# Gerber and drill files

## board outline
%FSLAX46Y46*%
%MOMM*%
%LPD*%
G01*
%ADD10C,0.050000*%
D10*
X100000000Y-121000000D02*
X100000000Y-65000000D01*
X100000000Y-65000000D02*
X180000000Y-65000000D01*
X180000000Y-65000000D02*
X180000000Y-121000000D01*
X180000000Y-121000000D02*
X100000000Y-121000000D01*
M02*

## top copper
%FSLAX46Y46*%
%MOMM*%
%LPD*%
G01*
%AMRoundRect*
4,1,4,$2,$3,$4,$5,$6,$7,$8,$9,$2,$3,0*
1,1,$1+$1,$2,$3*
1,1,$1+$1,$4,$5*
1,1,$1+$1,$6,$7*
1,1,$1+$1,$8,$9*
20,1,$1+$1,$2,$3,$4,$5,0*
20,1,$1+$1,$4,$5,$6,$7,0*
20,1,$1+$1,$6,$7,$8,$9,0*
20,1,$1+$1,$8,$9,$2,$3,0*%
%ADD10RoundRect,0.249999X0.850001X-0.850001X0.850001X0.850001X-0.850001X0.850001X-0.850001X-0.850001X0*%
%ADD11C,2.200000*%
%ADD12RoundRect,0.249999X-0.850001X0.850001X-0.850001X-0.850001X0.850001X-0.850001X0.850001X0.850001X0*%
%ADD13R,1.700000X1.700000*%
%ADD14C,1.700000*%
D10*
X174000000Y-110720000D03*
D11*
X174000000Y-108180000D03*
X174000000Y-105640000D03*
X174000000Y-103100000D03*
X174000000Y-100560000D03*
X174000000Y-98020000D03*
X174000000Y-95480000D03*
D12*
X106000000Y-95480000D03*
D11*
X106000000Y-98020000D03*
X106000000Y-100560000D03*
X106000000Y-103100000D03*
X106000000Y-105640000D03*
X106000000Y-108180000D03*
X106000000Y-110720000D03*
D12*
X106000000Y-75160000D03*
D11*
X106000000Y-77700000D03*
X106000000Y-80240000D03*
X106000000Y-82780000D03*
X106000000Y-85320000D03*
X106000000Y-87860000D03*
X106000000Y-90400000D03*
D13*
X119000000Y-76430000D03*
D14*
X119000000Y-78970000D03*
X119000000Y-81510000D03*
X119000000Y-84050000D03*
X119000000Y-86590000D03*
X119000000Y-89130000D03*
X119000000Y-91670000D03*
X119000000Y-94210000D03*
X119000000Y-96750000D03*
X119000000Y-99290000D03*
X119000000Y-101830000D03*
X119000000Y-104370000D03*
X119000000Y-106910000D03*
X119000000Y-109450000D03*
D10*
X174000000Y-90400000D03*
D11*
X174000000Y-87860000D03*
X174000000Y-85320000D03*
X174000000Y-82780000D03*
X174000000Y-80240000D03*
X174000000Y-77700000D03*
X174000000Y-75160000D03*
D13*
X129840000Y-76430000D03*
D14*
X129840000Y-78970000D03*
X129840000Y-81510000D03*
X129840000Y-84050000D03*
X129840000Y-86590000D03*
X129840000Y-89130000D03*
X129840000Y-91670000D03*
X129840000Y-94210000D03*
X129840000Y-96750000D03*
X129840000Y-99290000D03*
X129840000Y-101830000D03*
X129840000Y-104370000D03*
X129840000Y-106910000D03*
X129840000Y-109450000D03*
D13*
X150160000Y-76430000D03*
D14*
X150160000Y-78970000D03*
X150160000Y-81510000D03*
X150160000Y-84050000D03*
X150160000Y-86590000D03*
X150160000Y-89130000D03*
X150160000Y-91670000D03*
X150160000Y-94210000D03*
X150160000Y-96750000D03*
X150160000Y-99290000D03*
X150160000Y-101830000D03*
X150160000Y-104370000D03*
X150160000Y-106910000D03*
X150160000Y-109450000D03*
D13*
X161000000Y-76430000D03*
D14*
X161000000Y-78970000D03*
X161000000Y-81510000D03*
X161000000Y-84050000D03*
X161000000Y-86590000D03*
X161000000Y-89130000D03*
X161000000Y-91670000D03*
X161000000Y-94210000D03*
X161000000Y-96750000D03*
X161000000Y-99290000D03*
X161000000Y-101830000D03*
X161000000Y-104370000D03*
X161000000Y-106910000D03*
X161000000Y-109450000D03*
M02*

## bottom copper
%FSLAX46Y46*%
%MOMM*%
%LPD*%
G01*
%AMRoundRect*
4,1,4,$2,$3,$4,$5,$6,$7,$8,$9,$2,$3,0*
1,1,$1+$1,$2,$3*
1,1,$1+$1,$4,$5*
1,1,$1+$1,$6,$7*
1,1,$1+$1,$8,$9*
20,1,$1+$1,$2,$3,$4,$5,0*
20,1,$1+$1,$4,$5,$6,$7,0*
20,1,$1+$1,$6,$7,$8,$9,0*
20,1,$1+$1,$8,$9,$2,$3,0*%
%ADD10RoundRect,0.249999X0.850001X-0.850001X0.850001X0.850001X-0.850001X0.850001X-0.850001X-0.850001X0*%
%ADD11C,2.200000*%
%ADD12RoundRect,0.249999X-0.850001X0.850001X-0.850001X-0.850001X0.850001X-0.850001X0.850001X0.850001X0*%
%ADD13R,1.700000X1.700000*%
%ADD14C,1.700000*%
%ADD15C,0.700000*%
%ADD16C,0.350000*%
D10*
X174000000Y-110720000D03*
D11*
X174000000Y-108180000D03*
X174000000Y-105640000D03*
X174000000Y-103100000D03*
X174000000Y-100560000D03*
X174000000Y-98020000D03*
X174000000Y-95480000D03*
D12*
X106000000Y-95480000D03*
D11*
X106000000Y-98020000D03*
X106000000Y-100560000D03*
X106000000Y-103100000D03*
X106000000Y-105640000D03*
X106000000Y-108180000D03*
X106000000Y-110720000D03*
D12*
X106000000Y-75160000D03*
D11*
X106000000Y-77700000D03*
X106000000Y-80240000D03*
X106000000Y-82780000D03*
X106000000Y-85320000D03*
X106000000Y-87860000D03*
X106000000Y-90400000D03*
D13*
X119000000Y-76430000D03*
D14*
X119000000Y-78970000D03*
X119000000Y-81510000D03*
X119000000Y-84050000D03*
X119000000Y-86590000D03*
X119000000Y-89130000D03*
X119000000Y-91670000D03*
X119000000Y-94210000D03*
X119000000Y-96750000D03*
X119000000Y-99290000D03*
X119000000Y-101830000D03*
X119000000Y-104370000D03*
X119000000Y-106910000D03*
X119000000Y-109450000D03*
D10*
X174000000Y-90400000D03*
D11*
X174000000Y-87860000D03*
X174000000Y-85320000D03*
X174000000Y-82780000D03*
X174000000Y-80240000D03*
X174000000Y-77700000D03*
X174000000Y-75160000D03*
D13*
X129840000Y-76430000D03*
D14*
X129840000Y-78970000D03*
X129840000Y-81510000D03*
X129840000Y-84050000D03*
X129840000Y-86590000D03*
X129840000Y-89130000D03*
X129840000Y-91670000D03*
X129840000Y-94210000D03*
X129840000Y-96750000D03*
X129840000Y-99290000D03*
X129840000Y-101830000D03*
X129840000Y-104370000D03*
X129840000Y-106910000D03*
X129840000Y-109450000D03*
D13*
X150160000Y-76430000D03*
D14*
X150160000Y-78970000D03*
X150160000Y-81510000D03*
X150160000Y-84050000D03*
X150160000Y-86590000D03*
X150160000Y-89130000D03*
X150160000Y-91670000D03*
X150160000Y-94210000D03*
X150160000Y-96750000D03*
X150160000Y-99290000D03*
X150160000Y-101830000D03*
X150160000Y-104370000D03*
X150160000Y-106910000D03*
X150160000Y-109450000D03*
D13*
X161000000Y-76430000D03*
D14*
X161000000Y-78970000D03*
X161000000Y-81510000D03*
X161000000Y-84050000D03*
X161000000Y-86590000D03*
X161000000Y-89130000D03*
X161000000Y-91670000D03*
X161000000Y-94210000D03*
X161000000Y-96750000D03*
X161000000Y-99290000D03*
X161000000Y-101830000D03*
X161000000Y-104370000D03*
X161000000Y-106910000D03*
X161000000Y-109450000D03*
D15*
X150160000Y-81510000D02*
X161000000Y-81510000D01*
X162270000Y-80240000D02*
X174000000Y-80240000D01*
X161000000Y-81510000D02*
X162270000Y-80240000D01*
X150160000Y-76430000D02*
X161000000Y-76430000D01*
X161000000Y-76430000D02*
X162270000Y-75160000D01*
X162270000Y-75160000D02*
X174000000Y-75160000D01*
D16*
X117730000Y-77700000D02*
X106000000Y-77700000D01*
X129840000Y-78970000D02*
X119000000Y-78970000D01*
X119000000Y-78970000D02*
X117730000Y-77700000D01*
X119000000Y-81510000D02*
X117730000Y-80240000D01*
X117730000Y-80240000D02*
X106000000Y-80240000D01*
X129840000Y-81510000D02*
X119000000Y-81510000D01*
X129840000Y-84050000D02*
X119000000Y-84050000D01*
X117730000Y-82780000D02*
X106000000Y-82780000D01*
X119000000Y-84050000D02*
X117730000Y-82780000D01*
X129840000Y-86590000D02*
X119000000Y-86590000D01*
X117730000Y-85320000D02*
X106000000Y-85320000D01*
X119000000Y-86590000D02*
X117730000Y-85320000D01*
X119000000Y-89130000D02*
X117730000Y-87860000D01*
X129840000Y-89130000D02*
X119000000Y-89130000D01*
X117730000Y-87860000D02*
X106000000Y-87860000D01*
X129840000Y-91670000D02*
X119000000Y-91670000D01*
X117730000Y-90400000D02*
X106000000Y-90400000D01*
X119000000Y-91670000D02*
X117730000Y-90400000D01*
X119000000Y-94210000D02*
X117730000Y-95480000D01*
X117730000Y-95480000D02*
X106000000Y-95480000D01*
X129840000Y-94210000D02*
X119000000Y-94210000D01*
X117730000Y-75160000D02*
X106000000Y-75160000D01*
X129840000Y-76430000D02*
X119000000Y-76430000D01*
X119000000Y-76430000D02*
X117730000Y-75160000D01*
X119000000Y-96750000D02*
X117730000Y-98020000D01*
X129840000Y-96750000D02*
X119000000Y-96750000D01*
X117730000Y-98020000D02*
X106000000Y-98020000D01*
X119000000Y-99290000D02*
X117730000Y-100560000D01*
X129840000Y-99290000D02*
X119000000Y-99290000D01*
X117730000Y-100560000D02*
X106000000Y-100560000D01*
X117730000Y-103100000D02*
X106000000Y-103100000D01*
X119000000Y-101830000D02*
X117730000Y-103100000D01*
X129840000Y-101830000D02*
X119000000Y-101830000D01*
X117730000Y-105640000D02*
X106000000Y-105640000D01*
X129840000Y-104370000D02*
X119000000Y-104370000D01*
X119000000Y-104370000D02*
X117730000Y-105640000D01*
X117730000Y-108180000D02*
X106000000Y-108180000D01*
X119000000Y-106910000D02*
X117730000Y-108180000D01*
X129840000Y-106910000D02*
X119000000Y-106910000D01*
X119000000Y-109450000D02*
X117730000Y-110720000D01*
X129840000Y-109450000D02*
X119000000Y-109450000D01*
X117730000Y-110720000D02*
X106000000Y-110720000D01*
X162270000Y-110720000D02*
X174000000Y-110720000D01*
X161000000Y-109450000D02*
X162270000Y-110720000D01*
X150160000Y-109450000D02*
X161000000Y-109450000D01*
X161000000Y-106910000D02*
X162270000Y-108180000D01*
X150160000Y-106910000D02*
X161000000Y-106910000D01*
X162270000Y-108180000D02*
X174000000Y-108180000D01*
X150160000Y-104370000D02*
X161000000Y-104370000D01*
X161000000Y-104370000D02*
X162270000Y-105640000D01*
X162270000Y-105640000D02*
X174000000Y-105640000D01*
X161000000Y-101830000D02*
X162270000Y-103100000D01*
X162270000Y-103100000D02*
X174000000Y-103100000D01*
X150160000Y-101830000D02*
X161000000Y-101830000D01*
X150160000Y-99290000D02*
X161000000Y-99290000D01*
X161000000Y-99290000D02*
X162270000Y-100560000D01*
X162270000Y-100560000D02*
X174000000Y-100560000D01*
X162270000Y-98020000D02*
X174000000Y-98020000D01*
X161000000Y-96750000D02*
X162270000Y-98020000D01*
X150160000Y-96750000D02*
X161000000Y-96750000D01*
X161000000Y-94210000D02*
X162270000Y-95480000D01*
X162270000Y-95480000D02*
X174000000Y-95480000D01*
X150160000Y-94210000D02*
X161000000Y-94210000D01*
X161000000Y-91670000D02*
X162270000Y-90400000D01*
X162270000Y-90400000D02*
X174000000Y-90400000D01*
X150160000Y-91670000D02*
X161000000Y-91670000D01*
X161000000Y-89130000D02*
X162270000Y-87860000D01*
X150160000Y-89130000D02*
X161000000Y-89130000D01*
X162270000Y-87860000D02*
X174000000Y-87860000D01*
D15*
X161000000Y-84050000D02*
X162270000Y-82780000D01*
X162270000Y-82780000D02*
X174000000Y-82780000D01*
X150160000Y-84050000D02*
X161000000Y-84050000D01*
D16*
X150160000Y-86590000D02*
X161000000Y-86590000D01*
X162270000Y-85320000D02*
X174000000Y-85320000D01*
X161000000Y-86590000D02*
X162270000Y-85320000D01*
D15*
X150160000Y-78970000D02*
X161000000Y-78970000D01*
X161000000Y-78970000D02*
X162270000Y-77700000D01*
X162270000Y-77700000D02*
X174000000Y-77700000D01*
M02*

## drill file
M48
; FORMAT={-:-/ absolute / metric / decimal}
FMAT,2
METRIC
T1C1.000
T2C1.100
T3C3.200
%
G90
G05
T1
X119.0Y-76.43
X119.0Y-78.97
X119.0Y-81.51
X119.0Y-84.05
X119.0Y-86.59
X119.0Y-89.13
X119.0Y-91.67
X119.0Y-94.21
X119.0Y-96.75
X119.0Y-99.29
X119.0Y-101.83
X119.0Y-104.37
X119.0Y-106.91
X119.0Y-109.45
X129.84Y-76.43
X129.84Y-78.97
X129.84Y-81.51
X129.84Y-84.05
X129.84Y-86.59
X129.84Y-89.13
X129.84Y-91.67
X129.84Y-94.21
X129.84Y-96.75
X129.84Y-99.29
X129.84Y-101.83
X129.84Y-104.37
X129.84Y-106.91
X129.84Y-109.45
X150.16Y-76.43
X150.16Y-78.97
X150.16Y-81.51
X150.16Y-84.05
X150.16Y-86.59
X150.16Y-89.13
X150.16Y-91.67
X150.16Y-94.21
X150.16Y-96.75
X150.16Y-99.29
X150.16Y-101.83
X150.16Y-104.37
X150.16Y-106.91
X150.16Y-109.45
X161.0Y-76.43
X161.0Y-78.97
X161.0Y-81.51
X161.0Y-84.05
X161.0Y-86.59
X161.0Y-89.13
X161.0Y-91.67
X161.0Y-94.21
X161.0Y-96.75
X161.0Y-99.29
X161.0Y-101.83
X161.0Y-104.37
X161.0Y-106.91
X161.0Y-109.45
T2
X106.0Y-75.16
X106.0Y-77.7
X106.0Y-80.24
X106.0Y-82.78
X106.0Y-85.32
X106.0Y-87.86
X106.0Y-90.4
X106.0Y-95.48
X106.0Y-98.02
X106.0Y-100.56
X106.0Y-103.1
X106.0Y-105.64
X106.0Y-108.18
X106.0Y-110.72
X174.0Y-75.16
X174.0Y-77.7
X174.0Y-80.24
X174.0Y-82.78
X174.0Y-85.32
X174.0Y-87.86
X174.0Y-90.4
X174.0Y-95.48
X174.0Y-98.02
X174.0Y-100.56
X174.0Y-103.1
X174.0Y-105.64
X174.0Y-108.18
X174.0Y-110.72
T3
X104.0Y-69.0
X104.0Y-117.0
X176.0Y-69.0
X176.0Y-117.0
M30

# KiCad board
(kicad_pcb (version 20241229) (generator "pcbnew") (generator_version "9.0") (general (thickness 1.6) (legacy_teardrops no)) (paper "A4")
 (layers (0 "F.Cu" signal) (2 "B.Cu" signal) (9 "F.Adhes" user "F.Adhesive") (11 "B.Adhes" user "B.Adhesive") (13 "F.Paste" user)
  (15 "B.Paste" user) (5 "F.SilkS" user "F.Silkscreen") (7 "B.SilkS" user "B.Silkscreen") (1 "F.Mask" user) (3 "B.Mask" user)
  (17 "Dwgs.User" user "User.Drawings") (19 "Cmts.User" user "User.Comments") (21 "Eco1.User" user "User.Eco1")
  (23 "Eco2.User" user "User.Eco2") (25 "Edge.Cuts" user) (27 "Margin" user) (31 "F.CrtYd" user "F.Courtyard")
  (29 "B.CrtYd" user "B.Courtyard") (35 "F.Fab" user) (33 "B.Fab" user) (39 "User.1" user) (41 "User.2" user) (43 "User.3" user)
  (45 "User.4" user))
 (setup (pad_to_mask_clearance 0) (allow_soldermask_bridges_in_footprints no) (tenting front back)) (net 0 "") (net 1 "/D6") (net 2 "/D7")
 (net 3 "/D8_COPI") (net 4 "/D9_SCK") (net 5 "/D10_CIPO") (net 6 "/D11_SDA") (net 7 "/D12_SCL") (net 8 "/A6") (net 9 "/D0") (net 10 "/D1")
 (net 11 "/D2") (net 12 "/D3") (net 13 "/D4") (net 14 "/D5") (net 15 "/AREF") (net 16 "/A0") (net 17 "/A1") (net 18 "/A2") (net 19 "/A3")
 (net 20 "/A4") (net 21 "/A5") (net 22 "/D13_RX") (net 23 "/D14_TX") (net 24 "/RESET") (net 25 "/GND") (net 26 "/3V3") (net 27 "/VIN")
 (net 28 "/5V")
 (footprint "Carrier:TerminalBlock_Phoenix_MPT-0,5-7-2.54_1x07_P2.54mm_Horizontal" (layer "F.Cu") (at 174 110.72 90)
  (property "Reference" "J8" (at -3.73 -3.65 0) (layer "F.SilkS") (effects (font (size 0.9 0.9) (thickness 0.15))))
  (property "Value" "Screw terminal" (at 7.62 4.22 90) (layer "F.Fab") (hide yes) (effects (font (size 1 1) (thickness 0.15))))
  (pad "1" thru_hole roundrect (at 0 0 90) (size 2.2 2.2) (drill 1.1) (layers "*.Cu" "*.Mask") (remove_unused_layers no)
   (roundrect_rratio 0.113636) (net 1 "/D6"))
  (pad "2" thru_hole circle (at 2.54 0 90) (size 2.2 2.2) (drill 1.1) (layers "*.Cu" "*.Mask") (remove_unused_layers no) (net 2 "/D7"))
  (pad "3" thru_hole circle (at 5.08 0 90) (size 2.2 2.2) (drill 1.1) (layers "*.Cu" "*.Mask") (remove_unused_layers no) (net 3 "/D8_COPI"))
  (pad "4" thru_hole circle (at 7.62 0 90) (size 2.2 2.2) (drill 1.1) (layers "*.Cu" "*.Mask") (remove_unused_layers no) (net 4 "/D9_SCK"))
  (pad "5" thru_hole circle (at 10.16 0 90) (size 2.2 2.2) (drill 1.1) (layers "*.Cu" "*.Mask") (remove_unused_layers no)
   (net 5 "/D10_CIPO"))
  (pad "6" thru_hole circle (at 12.7 0 90) (size 2.2 2.2) (drill 1.1) (layers "*.Cu" "*.Mask") (remove_unused_layers no) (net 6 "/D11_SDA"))
  (pad "7" thru_hole circle (at 15.24 0 90) (size 2.2 2.2) (drill 1.1) (layers "*.Cu" "*.Mask") (remove_unused_layers no) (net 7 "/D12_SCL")))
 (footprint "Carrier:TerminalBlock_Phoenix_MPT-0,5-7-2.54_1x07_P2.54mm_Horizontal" (layer "F.Cu") (at 106 95.48 -90)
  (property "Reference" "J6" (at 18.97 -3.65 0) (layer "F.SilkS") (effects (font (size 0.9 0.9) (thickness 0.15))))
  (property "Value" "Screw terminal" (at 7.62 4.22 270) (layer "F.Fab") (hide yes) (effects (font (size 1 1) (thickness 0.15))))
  (pad "1" thru_hole roundrect (at 0 0 270) (size 2.2 2.2) (drill 1.1) (layers "*.Cu" "*.Mask") (remove_unused_layers no)
   (roundrect_rratio 0.113636) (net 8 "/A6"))
  (pad "2" thru_hole circle (at 2.54 0 270) (size 2.2 2.2) (drill 1.1) (layers "*.Cu" "*.Mask") (remove_unused_layers no) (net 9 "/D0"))
  (pad "3" thru_hole circle (at 5.08 0 270) (size 2.2 2.2) (drill 1.1) (layers "*.Cu" "*.Mask") (remove_unused_layers no) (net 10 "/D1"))
  (pad "4" thru_hole circle (at 7.62 0 270) (size 2.2 2.2) (drill 1.1) (layers "*.Cu" "*.Mask") (remove_unused_layers no) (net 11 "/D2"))
  (pad "5" thru_hole circle (at 10.16 0 270) (size 2.2 2.2) (drill 1.1) (layers "*.Cu" "*.Mask") (remove_unused_layers no) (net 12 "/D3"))
  (pad "6" thru_hole circle (at 12.7 0 270) (size 2.2 2.2) (drill 1.1) (layers "*.Cu" "*.Mask") (remove_unused_layers no) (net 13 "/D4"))
  (pad "7" thru_hole circle (at 15.24 0 270) (size 2.2 2.2) (drill 1.1) (layers "*.Cu" "*.Mask") (remove_unused_layers no) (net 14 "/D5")))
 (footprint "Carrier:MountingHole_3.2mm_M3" (layer "F.Cu") (at 176 117)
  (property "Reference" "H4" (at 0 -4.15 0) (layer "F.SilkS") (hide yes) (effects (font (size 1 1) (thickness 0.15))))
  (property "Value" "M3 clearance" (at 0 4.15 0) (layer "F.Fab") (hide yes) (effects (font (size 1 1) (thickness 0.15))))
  (pad "" np_thru_hole circle (at 0 0) (size 3.2 3.2) (drill 3.2) (layers "*.Cu" "*.Mask")))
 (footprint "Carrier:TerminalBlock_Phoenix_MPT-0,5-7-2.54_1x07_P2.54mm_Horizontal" (layer "F.Cu") (at 106 75.16 -90)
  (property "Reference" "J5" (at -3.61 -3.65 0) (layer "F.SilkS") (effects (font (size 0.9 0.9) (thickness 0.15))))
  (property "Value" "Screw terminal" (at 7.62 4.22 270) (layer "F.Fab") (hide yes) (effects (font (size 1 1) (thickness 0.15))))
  (pad "1" thru_hole roundrect (at 0 0 270) (size 2.2 2.2) (drill 1.1) (layers "*.Cu" "*.Mask") (remove_unused_layers no)
   (roundrect_rratio 0.113636) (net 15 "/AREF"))
  (pad "2" thru_hole circle (at 2.54 0 270) (size 2.2 2.2) (drill 1.1) (layers "*.Cu" "*.Mask") (remove_unused_layers no) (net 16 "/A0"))
  (pad "3" thru_hole circle (at 5.08 0 270) (size 2.2 2.2) (drill 1.1) (layers "*.Cu" "*.Mask") (remove_unused_layers no) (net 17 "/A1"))
  (pad "4" thru_hole circle (at 7.62 0 270) (size 2.2 2.2) (drill 1.1) (layers "*.Cu" "*.Mask") (remove_unused_layers no) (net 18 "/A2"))
  (pad "5" thru_hole circle (at 10.16 0 270) (size 2.2 2.2) (drill 1.1) (layers "*.Cu" "*.Mask") (remove_unused_layers no) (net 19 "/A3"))
  (pad "6" thru_hole circle (at 12.7 0 270) (size 2.2 2.2) (drill 1.1) (layers "*.Cu" "*.Mask") (remove_unused_layers no) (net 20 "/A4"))
  (pad "7" thru_hole circle (at 15.24 0 270) (size 2.2 2.2) (drill 1.1) (layers "*.Cu" "*.Mask") (remove_unused_layers no) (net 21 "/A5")))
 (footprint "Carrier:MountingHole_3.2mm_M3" (layer "F.Cu") (at 176 69)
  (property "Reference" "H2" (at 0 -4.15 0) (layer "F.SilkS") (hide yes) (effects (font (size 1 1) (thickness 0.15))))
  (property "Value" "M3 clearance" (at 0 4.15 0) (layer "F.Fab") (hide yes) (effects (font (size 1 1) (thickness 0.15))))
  (pad "" np_thru_hole circle (at 0 0) (size 3.2 3.2) (drill 3.2) (layers "*.Cu" "*.Mask")))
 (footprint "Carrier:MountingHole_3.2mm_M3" (layer "F.Cu") (at 104 69)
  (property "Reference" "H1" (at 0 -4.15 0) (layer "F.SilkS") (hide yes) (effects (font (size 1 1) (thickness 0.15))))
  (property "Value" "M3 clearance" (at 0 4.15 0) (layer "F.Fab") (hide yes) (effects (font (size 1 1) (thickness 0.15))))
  (pad "" np_thru_hole circle (at 0 0) (size 3.2 3.2) (drill 3.2) (layers "*.Cu" "*.Mask")))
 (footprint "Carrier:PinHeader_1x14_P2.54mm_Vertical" (layer "F.Cu") (at 119 76.43)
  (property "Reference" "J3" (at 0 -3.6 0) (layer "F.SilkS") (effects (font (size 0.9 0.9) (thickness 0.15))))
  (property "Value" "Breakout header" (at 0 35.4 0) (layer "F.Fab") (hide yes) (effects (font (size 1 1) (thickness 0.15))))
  (pad "1" thru_hole rect (at 0 0) (size 1.7 1.7) (drill 1) (layers "*.Cu" "*.Mask") (remove_unused_layers no) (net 15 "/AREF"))
  (pad "2" thru_hole circle (at 0 2.54) (size 1.7 1.7) (drill 1) (layers "*.Cu" "*.Mask") (remove_unused_layers no) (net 16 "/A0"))
  (pad "3" thru_hole circle (at 0 5.08) (size 1.7 1.7) (drill 1) (layers "*.Cu" "*.Mask") (remove_unused_layers no) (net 17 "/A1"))
  (pad "4" thru_hole circle (at 0 7.62) (size 1.7 1.7) (drill 1) (layers "*.Cu" "*.Mask") (remove_unused_layers no) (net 18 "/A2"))
  (pad "5" thru_hole circle (at 0 10.16) (size 1.7 1.7) (drill 1) (layers "*.Cu" "*.Mask") (remove_unused_layers no) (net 19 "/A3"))
  (pad "6" thru_hole circle (at 0 12.7) (size 1.7 1.7) (drill 1) (layers "*.Cu" "*.Mask") (remove_unused_layers no) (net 20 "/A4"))
  (pad "7" thru_hole circle (at 0 15.24) (size 1.7 1.7) (drill 1) (layers "*.Cu" "*.Mask") (remove_unused_layers no) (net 21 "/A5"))
  (pad "8" thru_hole circle (at 0 17.78) (size 1.7 1.7) (drill 1) (layers "*.Cu" "*.Mask") (remove_unused_layers no) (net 8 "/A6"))
  (pad "9" thru_hole circle (at 0 20.32) (size 1.7 1.7) (drill 1) (layers "*.Cu" "*.Mask") (remove_unused_layers no) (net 9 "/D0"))
  (pad "10" thru_hole circle (at 0 22.86) (size 1.7 1.7) (drill 1) (layers "*.Cu" "*.Mask") (remove_unused_layers no) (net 10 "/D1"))
  (pad "11" thru_hole circle (at 0 25.4) (size 1.7 1.7) (drill 1) (layers "*.Cu" "*.Mask") (remove_unused_layers no) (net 11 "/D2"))
  (pad "12" thru_hole circle (at 0 27.94) (size 1.7 1.7) (drill 1) (layers "*.Cu" "*.Mask") (remove_unused_layers no) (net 12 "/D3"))
  (pad "13" thru_hole circle (at 0 30.48) (size 1.7 1.7) (drill 1) (layers "*.Cu" "*.Mask") (remove_unused_layers no) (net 13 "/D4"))
  (pad "14" thru_hole circle (at 0 33.02) (size 1.7 1.7) (drill 1) (layers "*.Cu" "*.Mask") (remove_unused_layers no) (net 14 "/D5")))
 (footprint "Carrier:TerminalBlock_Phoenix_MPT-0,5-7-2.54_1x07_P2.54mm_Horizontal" (layer "F.Cu") (at 174 90.4 90)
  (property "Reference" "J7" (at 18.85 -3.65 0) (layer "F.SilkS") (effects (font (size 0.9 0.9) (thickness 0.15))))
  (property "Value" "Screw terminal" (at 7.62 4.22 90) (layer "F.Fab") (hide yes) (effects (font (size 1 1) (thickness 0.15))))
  (pad "1" thru_hole roundrect (at 0 0 90) (size 2.2 2.2) (drill 1.1) (layers "*.Cu" "*.Mask") (remove_unused_layers no)
   (roundrect_rratio 0.113636) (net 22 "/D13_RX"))
  (pad "2" thru_hole circle (at 2.54 0 90) (size 2.2 2.2) (drill 1.1) (layers "*.Cu" "*.Mask") (remove_unused_layers no) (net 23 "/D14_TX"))
  (pad "3" thru_hole circle (at 5.08 0 90) (size 2.2 2.2) (drill 1.1) (layers "*.Cu" "*.Mask") (remove_unused_layers no) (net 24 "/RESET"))
  (pad "4" thru_hole circle (at 7.62 0 90) (size 2.2 2.2) (drill 1.1) (layers "*.Cu" "*.Mask") (remove_unused_layers no) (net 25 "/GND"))
  (pad "5" thru_hole circle (at 10.16 0 90) (size 2.2 2.2) (drill 1.1) (layers "*.Cu" "*.Mask") (remove_unused_layers no) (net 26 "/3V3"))
  (pad "6" thru_hole circle (at 12.7 0 90) (size 2.2 2.2) (drill 1.1) (layers "*.Cu" "*.Mask") (remove_unused_layers no) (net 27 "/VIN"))
  (pad "7" thru_hole circle (at 15.24 0 90) (size 2.2 2.2) (drill 1.1) (layers "*.Cu" "*.Mask") (remove_unused_layers no) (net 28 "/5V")))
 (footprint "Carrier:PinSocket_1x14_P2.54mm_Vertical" (layer "F.Cu") (at 129.84 76.43)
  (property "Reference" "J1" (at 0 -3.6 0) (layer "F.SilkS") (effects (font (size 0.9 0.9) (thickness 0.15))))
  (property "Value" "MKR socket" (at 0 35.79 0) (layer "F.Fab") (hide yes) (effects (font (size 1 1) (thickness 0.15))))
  (pad "1" thru_hole rect (at 0 0) (size 1.7 1.7) (drill 1) (layers "*.Cu" "*.Mask") (remove_unused_layers no) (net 15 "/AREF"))
  (pad "2" thru_hole circle (at 0 2.54) (size 1.7 1.7) (drill 1) (layers "*.Cu" "*.Mask") (remove_unused_layers no) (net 16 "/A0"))
  (pad "3" thru_hole circle (at 0 5.08) (size 1.7 1.7) (drill 1) (layers "*.Cu" "*.Mask") (remove_unused_layers no) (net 17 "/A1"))
  (pad "4" thru_hole circle (at 0 7.62) (size 1.7 1.7) (drill 1) (layers "*.Cu" "*.Mask") (remove_unused_layers no) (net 18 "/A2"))
  (pad "5" thru_hole circle (at 0 10.16) (size 1.7 1.7) (drill 1) (layers "*.Cu" "*.Mask") (remove_unused_layers no) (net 19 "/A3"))
  (pad "6" thru_hole circle (at 0 12.7) (size 1.7 1.7) (drill 1) (layers "*.Cu" "*.Mask") (remove_unused_layers no) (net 20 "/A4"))
  (pad "7" thru_hole circle (at 0 15.24) (size 1.7 1.7) (drill 1) (layers "*.Cu" "*.Mask") (remove_unused_layers no) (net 21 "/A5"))
  (pad "8" thru_hole circle (at 0 17.78) (size 1.7 1.7) (drill 1) (layers "*.Cu" "*.Mask") (remove_unused_layers no) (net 8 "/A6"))
  (pad "9" thru_hole circle (at 0 20.32) (size 1.7 1.7) (drill 1) (layers "*.Cu" "*.Mask") (remove_unused_layers no) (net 9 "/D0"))
  (pad "10" thru_hole circle (at 0 22.86) (size 1.7 1.7) (drill 1) (layers "*.Cu" "*.Mask") (remove_unused_layers no) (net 10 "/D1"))
  (pad "11" thru_hole circle (at 0 25.4) (size 1.7 1.7) (drill 1) (layers "*.Cu" "*.Mask") (remove_unused_layers no) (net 11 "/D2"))
  (pad "12" thru_hole circle (at 0 27.94) (size 1.7 1.7) (drill 1) (layers "*.Cu" "*.Mask") (remove_unused_layers no) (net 12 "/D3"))
  (pad "13" thru_hole circle (at 0 30.48) (size 1.7 1.7) (drill 1) (layers "*.Cu" "*.Mask") (remove_unused_layers no) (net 13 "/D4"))
  (pad "14" thru_hole circle (at 0 33.02) (size 1.7 1.7) (drill 1) (layers "*.Cu" "*.Mask") (remove_unused_layers no) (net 14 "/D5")))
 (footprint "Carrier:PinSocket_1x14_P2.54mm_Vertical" (layer "F.Cu") (at 150.16 76.43)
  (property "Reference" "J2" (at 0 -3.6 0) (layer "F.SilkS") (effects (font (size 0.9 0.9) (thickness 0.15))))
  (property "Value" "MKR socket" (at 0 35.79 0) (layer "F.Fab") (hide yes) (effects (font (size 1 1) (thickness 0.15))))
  (pad "1" thru_hole rect (at 0 0) (size 1.7 1.7) (drill 1) (layers "*.Cu" "*.Mask") (remove_unused_layers no) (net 28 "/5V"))
  (pad "2" thru_hole circle (at 0 2.54) (size 1.7 1.7) (drill 1) (layers "*.Cu" "*.Mask") (remove_unused_layers no) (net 27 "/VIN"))
  (pad "3" thru_hole circle (at 0 5.08) (size 1.7 1.7) (drill 1) (layers "*.Cu" "*.Mask") (remove_unused_layers no) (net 26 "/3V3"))
  (pad "4" thru_hole circle (at 0 7.62) (size 1.7 1.7) (drill 1) (layers "*.Cu" "*.Mask") (remove_unused_layers no) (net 25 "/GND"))
  (pad "5" thru_hole circle (at 0 10.16) (size 1.7 1.7) (drill 1) (layers "*.Cu" "*.Mask") (remove_unused_layers no) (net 24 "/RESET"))
  (pad "6" thru_hole circle (at 0 12.7) (size 1.7 1.7) (drill 1) (layers "*.Cu" "*.Mask") (remove_unused_layers no) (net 23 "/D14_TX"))
  (pad "7" thru_hole circle (at 0 15.24) (size 1.7 1.7) (drill 1) (layers "*.Cu" "*.Mask") (remove_unused_layers no) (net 22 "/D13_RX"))
  (pad "8" thru_hole circle (at 0 17.78) (size 1.7 1.7) (drill 1) (layers "*.Cu" "*.Mask") (remove_unused_layers no) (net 7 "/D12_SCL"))
  (pad "9" thru_hole circle (at 0 20.32) (size 1.7 1.7) (drill 1) (layers "*.Cu" "*.Mask") (remove_unused_layers no) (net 6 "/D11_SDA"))
  (pad "10" thru_hole circle (at 0 22.86) (size 1.7 1.7) (drill 1) (layers "*.Cu" "*.Mask") (remove_unused_layers no) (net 5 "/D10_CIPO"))
  (pad "11" thru_hole circle (at 0 25.4) (size 1.7 1.7) (drill 1) (layers "*.Cu" "*.Mask") (remove_unused_layers no) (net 4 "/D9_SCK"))
  (pad "12" thru_hole circle (at 0 27.94) (size 1.7 1.7) (drill 1) (layers "*.Cu" "*.Mask") (remove_unused_layers no) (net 3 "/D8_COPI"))
  (pad "13" thru_hole circle (at 0 30.48) (size 1.7 1.7) (drill 1) (layers "*.Cu" "*.Mask") (remove_unused_layers no) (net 2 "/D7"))
  (pad "14" thru_hole circle (at 0 33.02) (size 1.7 1.7) (drill 1) (layers "*.Cu" "*.Mask") (remove_unused_layers no) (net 1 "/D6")))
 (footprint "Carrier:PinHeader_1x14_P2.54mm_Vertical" (layer "F.Cu") (at 161 76.43)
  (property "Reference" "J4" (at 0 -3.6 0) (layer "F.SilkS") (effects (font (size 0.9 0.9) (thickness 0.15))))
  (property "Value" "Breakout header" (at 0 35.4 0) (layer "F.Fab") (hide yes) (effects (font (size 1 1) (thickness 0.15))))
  (pad "1" thru_hole rect (at 0 0) (size 1.7 1.7) (drill 1) (layers "*.Cu" "*.Mask") (remove_unused_layers no) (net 28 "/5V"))
  (pad "2" thru_hole circle (at 0 2.54) (size 1.7 1.7) (drill 1) (layers "*.Cu" "*.Mask") (remove_unused_layers no) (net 27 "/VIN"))
  (pad "3" thru_hole circle (at 0 5.08) (size 1.7 1.7) (drill 1) (layers "*.Cu" "*.Mask") (remove_unused_layers no) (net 26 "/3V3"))
  (pad "4" thru_hole circle (at 0 7.62) (size 1.7 1.7) (drill 1) (layers "*.Cu" "*.Mask") (remove_unused_layers no) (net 25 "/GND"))
  (pad "5" thru_hole circle (at 0 10.16) (size 1.7 1.7) (drill 1) (layers "*.Cu" "*.Mask") (remove_unused_layers no) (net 24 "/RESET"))
  (pad "6" thru_hole circle (at 0 12.7) (size 1.7 1.7) (drill 1) (layers "*.Cu" "*.Mask") (remove_unused_layers no) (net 23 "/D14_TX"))
  (pad "7" thru_hole circle (at 0 15.24) (size 1.7 1.7) (drill 1) (layers "*.Cu" "*.Mask") (remove_unused_layers no) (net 22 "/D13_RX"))
  (pad "8" thru_hole circle (at 0 17.78) (size 1.7 1.7) (drill 1) (layers "*.Cu" "*.Mask") (remove_unused_layers no) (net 7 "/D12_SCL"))
  (pad "9" thru_hole circle (at 0 20.32) (size 1.7 1.7) (drill 1) (layers "*.Cu" "*.Mask") (remove_unused_layers no) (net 6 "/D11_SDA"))
  (pad "10" thru_hole circle (at 0 22.86) (size 1.7 1.7) (drill 1) (layers "*.Cu" "*.Mask") (remove_unused_layers no) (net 5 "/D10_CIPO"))
  (pad "11" thru_hole circle (at 0 25.4) (size 1.7 1.7) (drill 1) (layers "*.Cu" "*.Mask") (remove_unused_layers no) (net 4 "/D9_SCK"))
  (pad "12" thru_hole circle (at 0 27.94) (size 1.7 1.7) (drill 1) (layers "*.Cu" "*.Mask") (remove_unused_layers no) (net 3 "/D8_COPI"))
  (pad "13" thru_hole circle (at 0 30.48) (size 1.7 1.7) (drill 1) (layers "*.Cu" "*.Mask") (remove_unused_layers no) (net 2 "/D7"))
  (pad "14" thru_hole circle (at 0 33.02) (size 1.7 1.7) (drill 1) (layers "*.Cu" "*.Mask") (remove_unused_layers no) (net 1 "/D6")))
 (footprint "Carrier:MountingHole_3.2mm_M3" (layer "F.Cu") (at 104 117)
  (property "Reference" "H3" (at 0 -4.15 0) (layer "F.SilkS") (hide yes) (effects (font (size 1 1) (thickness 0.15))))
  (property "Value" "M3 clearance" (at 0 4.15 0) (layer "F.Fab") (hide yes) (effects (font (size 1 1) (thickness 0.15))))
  (pad "" np_thru_hole circle (at 0 0) (size 3.2 3.2) (drill 3.2) (layers "*.Cu" "*.Mask")))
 (gr_line (start 100 121) (end 100 65) (stroke (width 0.05) (type default)) (layer "Edge.Cuts"))
 (gr_line (start 100 65) (end 180 65) (stroke (width 0.05) (type default)) (layer "Edge.Cuts"))
 (gr_line (start 180 65) (end 180 121) (stroke (width 0.05) (type default)) (layer "Edge.Cuts"))
 (gr_line (start 180 121) (end 100 121) (stroke (width 0.05) (type default)) (layer "Edge.Cuts"))
 (segment (start 150.16 81.51) (end 161 81.51) (width 0.7) (layer "B.Cu") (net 26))
 (segment (start 162.27 80.24) (end 174 80.24) (width 0.7) (layer "B.Cu") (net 26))
 (segment (start 161 81.51) (end 162.27 80.24) (width 0.7) (layer "B.Cu") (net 26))
 (segment (start 150.16 76.43) (end 161 76.43) (width 0.7) (layer "B.Cu") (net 28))
 (segment (start 161 76.43) (end 162.27 75.16) (width 0.7) (layer "B.Cu") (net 28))
 (segment (start 162.27 75.16) (end 174 75.16) (width 0.7) (layer "B.Cu") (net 28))
 (segment (start 117.73 77.7) (end 106 77.7) (width 0.35) (layer "B.Cu") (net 16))
 (segment (start 129.84 78.97) (end 119 78.97) (width 0.35) (layer "B.Cu") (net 16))
 (segment (start 119 78.97) (end 117.73 77.7) (width 0.35) (layer "B.Cu") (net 16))
 (segment (start 119 81.51) (end 117.73 80.24) (width 0.35) (layer "B.Cu") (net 17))
 (segment (start 117.73 80.24) (end 106 80.24) (width 0.35) (layer "B.Cu") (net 17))
 (segment (start 129.84 81.51) (end 119 81.51) (width 0.35) (layer "B.Cu") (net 17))
 (segment (start 129.84 84.05) (end 119 84.05) (width 0.35) (layer "B.Cu") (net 18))
 (segment (start 117.73 82.78) (end 106 82.78) (width 0.35) (layer "B.Cu") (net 18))
 (segment (start 119 84.05) (end 117.73 82.78) (width 0.35) (layer "B.Cu") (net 18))
 (segment (start 129.84 86.59) (end 119 86.59) (width 0.35) (layer "B.Cu") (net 19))
 (segment (start 117.73 85.32) (end 106 85.32) (width 0.35) (layer "B.Cu") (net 19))
 (segment (start 119 86.59) (end 117.73 85.32) (width 0.35) (layer "B.Cu") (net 19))
 (segment (start 119 89.13) (end 117.73 87.86) (width 0.35) (layer "B.Cu") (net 20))
 (segment (start 129.84 89.13) (end 119 89.13) (width 0.35) (layer "B.Cu") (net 20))
 (segment (start 117.73 87.86) (end 106 87.86) (width 0.35) (layer "B.Cu") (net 20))
 (segment (start 129.84 91.67) (end 119 91.67) (width 0.35) (layer "B.Cu") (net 21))
 (segment (start 117.73 90.4) (end 106 90.4) (width 0.35) (layer "B.Cu") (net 21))
 (segment (start 119 91.67) (end 117.73 90.4) (width 0.35) (layer "B.Cu") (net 21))
 (segment (start 119 94.21) (end 117.73 95.48) (width 0.35) (layer "B.Cu") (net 8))
 (segment (start 117.73 95.48) (end 106 95.48) (width 0.35) (layer "B.Cu") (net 8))
 (segment (start 129.84 94.21) (end 119 94.21) (width 0.35) (layer "B.Cu") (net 8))
 (segment (start 117.73 75.16) (end 106 75.16) (width 0.35) (layer "B.Cu") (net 15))
 (segment (start 129.84 76.43) (end 119 76.43) (width 0.35) (layer "B.Cu") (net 15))
 (segment (start 119 76.43) (end 117.73 75.16) (width 0.35) (layer "B.Cu") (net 15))
 (segment (start 119 96.75) (end 117.73 98.02) (width 0.35) (layer "B.Cu") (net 9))
 (segment (start 129.84 96.75) (end 119 96.75) (width 0.35) (layer "B.Cu") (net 9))
 (segment (start 117.73 98.02) (end 106 98.02) (width 0.35) (layer "B.Cu") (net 9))
 (segment (start 119 99.29) (end 117.73 100.56) (width 0.35) (layer "B.Cu") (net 10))
 (segment (start 129.84 99.29) (end 119 99.29) (width 0.35) (layer "B.Cu") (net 10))
 (segment (start 117.73 100.56) (end 106 100.56) (width 0.35) (layer "B.Cu") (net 10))
 (segment (start 117.73 103.1) (end 106 103.1) (width 0.35) (layer "B.Cu") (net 11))
 (segment (start 119 101.83) (end 117.73 103.1) (width 0.35) (layer "B.Cu") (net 11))
 (segment (start 129.84 101.83) (end 119 101.83) (width 0.35) (layer "B.Cu") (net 11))
 (segment (start 117.73 105.64) (end 106 105.64) (width 0.35) (layer "B.Cu") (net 12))
 (segment (start 129.84 104.37) (end 119 104.37) (width 0.35) (layer "B.Cu") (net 12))
 (segment (start 119 104.37) (end 117.73 105.64) (width 0.35) (layer "B.Cu") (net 12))
 (segment (start 117.73 108.18) (end 106 108.18) (width 0.35) (layer "B.Cu") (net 13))
 (segment (start 119 106.91) (end 117.73 108.18) (width 0.35) (layer "B.Cu") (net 13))
 (segment (start 129.84 106.91) (end 119 106.91) (width 0.35) (layer "B.Cu") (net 13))
 (segment (start 119 109.45) (end 117.73 110.72) (width 0.35) (layer "B.Cu") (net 14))
 (segment (start 129.84 109.45) (end 119 109.45) (width 0.35) (layer "B.Cu") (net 14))
 (segment (start 117.73 110.72) (end 106 110.72) (width 0.35) (layer "B.Cu") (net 14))
 (segment (start 162.27 110.72) (end 174 110.72) (width 0.35) (layer "B.Cu") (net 1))
 (segment (start 161 109.45) (end 162.27 110.72) (width 0.35) (layer "B.Cu") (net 1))
 (segment (start 150.16 109.45) (end 161 109.45) (width 0.35) (layer "B.Cu") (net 1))
 (segment (start 161 106.91) (end 162.27 108.18) (width 0.35) (layer "B.Cu") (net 2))
 (segment (start 150.16 106.91) (end 161 106.91) (width 0.35) (layer "B.Cu") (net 2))
 (segment (start 162.27 108.18) (end 174 108.18) (width 0.35) (layer "B.Cu") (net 2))
 (segment (start 150.16 104.37) (end 161 104.37) (width 0.35) (layer "B.Cu") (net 3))
 (segment (start 161 104.37) (end 162.27 105.64) (width 0.35) (layer "B.Cu") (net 3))
 (segment (start 162.27 105.64) (end 174 105.64) (width 0.35) (layer "B.Cu") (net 3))
 (segment (start 161 101.83) (end 162.27 103.1) (width 0.35) (layer "B.Cu") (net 4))
 (segment (start 162.27 103.1) (end 174 103.1) (width 0.35) (layer "B.Cu") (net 4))
 (segment (start 150.16 101.83) (end 161 101.83) (width 0.35) (layer "B.Cu") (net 4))
 (segment (start 150.16 99.29) (end 161 99.29) (width 0.35) (layer "B.Cu") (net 5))
 (segment (start 161 99.29) (end 162.27 100.56) (width 0.35) (layer "B.Cu") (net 5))
 (segment (start 162.27 100.56) (end 174 100.56) (width 0.35) (layer "B.Cu") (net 5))
 (segment (start 162.27 98.02) (end 174 98.02) (width 0.35) (layer "B.Cu") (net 6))
 (segment (start 161 96.75) (end 162.27 98.02) (width 0.35) (layer "B.Cu") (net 6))
 (segment (start 150.16 96.75) (end 161 96.75) (width 0.35) (layer "B.Cu") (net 6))
 (segment (start 161 94.21) (end 162.27 95.48) (width 0.35) (layer "B.Cu") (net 7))
 (segment (start 162.27 95.48) (end 174 95.48) (width 0.35) (layer "B.Cu") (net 7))
 (segment (start 150.16 94.21) (end 161 94.21) (width 0.35) (layer "B.Cu") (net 7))
 (segment (start 161 91.67) (end 162.27 90.4) (width 0.35) (layer "B.Cu") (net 22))
 (segment (start 162.27 90.4) (end 174 90.4) (width 0.35) (layer "B.Cu") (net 22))
 (segment (start 150.16 91.67) (end 161 91.67) (width 0.35) (layer "B.Cu") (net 22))
 (segment (start 161 89.13) (end 162.27 87.86) (width 0.35) (layer "B.Cu") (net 23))
 (segment (start 150.16 89.13) (end 161 89.13) (width 0.35) (layer "B.Cu") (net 23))
 (segment (start 162.27 87.86) (end 174 87.86) (width 0.35) (layer "B.Cu") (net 23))
 (segment (start 161 84.05) (end 162.27 82.78) (width 0.7) (layer "B.Cu") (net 25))
 (segment (start 162.27 82.78) (end 174 82.78) (width 0.7) (layer "B.Cu") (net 25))
 (segment (start 150.16 84.05) (end 161 84.05) (width 0.7) (layer "B.Cu") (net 25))
 (segment (start 150.16 86.59) (end 161 86.59) (width 0.35) (layer "B.Cu") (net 24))
 (segment (start 162.27 85.32) (end 174 85.32) (width 0.35) (layer "B.Cu") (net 24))
 (segment (start 161 86.59) (end 162.27 85.32) (width 0.35) (layer "B.Cu") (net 24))
 (segment (start 150.16 78.97) (end 161 78.97) (width 0.7) (layer "B.Cu") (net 27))
 (segment (start 161 78.97) (end 162.27 77.7) (width 0.7) (layer "B.Cu") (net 27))
 (segment (start 162.27 77.7) (end 174 77.7) (width 0.7) (layer "B.Cu") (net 27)))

